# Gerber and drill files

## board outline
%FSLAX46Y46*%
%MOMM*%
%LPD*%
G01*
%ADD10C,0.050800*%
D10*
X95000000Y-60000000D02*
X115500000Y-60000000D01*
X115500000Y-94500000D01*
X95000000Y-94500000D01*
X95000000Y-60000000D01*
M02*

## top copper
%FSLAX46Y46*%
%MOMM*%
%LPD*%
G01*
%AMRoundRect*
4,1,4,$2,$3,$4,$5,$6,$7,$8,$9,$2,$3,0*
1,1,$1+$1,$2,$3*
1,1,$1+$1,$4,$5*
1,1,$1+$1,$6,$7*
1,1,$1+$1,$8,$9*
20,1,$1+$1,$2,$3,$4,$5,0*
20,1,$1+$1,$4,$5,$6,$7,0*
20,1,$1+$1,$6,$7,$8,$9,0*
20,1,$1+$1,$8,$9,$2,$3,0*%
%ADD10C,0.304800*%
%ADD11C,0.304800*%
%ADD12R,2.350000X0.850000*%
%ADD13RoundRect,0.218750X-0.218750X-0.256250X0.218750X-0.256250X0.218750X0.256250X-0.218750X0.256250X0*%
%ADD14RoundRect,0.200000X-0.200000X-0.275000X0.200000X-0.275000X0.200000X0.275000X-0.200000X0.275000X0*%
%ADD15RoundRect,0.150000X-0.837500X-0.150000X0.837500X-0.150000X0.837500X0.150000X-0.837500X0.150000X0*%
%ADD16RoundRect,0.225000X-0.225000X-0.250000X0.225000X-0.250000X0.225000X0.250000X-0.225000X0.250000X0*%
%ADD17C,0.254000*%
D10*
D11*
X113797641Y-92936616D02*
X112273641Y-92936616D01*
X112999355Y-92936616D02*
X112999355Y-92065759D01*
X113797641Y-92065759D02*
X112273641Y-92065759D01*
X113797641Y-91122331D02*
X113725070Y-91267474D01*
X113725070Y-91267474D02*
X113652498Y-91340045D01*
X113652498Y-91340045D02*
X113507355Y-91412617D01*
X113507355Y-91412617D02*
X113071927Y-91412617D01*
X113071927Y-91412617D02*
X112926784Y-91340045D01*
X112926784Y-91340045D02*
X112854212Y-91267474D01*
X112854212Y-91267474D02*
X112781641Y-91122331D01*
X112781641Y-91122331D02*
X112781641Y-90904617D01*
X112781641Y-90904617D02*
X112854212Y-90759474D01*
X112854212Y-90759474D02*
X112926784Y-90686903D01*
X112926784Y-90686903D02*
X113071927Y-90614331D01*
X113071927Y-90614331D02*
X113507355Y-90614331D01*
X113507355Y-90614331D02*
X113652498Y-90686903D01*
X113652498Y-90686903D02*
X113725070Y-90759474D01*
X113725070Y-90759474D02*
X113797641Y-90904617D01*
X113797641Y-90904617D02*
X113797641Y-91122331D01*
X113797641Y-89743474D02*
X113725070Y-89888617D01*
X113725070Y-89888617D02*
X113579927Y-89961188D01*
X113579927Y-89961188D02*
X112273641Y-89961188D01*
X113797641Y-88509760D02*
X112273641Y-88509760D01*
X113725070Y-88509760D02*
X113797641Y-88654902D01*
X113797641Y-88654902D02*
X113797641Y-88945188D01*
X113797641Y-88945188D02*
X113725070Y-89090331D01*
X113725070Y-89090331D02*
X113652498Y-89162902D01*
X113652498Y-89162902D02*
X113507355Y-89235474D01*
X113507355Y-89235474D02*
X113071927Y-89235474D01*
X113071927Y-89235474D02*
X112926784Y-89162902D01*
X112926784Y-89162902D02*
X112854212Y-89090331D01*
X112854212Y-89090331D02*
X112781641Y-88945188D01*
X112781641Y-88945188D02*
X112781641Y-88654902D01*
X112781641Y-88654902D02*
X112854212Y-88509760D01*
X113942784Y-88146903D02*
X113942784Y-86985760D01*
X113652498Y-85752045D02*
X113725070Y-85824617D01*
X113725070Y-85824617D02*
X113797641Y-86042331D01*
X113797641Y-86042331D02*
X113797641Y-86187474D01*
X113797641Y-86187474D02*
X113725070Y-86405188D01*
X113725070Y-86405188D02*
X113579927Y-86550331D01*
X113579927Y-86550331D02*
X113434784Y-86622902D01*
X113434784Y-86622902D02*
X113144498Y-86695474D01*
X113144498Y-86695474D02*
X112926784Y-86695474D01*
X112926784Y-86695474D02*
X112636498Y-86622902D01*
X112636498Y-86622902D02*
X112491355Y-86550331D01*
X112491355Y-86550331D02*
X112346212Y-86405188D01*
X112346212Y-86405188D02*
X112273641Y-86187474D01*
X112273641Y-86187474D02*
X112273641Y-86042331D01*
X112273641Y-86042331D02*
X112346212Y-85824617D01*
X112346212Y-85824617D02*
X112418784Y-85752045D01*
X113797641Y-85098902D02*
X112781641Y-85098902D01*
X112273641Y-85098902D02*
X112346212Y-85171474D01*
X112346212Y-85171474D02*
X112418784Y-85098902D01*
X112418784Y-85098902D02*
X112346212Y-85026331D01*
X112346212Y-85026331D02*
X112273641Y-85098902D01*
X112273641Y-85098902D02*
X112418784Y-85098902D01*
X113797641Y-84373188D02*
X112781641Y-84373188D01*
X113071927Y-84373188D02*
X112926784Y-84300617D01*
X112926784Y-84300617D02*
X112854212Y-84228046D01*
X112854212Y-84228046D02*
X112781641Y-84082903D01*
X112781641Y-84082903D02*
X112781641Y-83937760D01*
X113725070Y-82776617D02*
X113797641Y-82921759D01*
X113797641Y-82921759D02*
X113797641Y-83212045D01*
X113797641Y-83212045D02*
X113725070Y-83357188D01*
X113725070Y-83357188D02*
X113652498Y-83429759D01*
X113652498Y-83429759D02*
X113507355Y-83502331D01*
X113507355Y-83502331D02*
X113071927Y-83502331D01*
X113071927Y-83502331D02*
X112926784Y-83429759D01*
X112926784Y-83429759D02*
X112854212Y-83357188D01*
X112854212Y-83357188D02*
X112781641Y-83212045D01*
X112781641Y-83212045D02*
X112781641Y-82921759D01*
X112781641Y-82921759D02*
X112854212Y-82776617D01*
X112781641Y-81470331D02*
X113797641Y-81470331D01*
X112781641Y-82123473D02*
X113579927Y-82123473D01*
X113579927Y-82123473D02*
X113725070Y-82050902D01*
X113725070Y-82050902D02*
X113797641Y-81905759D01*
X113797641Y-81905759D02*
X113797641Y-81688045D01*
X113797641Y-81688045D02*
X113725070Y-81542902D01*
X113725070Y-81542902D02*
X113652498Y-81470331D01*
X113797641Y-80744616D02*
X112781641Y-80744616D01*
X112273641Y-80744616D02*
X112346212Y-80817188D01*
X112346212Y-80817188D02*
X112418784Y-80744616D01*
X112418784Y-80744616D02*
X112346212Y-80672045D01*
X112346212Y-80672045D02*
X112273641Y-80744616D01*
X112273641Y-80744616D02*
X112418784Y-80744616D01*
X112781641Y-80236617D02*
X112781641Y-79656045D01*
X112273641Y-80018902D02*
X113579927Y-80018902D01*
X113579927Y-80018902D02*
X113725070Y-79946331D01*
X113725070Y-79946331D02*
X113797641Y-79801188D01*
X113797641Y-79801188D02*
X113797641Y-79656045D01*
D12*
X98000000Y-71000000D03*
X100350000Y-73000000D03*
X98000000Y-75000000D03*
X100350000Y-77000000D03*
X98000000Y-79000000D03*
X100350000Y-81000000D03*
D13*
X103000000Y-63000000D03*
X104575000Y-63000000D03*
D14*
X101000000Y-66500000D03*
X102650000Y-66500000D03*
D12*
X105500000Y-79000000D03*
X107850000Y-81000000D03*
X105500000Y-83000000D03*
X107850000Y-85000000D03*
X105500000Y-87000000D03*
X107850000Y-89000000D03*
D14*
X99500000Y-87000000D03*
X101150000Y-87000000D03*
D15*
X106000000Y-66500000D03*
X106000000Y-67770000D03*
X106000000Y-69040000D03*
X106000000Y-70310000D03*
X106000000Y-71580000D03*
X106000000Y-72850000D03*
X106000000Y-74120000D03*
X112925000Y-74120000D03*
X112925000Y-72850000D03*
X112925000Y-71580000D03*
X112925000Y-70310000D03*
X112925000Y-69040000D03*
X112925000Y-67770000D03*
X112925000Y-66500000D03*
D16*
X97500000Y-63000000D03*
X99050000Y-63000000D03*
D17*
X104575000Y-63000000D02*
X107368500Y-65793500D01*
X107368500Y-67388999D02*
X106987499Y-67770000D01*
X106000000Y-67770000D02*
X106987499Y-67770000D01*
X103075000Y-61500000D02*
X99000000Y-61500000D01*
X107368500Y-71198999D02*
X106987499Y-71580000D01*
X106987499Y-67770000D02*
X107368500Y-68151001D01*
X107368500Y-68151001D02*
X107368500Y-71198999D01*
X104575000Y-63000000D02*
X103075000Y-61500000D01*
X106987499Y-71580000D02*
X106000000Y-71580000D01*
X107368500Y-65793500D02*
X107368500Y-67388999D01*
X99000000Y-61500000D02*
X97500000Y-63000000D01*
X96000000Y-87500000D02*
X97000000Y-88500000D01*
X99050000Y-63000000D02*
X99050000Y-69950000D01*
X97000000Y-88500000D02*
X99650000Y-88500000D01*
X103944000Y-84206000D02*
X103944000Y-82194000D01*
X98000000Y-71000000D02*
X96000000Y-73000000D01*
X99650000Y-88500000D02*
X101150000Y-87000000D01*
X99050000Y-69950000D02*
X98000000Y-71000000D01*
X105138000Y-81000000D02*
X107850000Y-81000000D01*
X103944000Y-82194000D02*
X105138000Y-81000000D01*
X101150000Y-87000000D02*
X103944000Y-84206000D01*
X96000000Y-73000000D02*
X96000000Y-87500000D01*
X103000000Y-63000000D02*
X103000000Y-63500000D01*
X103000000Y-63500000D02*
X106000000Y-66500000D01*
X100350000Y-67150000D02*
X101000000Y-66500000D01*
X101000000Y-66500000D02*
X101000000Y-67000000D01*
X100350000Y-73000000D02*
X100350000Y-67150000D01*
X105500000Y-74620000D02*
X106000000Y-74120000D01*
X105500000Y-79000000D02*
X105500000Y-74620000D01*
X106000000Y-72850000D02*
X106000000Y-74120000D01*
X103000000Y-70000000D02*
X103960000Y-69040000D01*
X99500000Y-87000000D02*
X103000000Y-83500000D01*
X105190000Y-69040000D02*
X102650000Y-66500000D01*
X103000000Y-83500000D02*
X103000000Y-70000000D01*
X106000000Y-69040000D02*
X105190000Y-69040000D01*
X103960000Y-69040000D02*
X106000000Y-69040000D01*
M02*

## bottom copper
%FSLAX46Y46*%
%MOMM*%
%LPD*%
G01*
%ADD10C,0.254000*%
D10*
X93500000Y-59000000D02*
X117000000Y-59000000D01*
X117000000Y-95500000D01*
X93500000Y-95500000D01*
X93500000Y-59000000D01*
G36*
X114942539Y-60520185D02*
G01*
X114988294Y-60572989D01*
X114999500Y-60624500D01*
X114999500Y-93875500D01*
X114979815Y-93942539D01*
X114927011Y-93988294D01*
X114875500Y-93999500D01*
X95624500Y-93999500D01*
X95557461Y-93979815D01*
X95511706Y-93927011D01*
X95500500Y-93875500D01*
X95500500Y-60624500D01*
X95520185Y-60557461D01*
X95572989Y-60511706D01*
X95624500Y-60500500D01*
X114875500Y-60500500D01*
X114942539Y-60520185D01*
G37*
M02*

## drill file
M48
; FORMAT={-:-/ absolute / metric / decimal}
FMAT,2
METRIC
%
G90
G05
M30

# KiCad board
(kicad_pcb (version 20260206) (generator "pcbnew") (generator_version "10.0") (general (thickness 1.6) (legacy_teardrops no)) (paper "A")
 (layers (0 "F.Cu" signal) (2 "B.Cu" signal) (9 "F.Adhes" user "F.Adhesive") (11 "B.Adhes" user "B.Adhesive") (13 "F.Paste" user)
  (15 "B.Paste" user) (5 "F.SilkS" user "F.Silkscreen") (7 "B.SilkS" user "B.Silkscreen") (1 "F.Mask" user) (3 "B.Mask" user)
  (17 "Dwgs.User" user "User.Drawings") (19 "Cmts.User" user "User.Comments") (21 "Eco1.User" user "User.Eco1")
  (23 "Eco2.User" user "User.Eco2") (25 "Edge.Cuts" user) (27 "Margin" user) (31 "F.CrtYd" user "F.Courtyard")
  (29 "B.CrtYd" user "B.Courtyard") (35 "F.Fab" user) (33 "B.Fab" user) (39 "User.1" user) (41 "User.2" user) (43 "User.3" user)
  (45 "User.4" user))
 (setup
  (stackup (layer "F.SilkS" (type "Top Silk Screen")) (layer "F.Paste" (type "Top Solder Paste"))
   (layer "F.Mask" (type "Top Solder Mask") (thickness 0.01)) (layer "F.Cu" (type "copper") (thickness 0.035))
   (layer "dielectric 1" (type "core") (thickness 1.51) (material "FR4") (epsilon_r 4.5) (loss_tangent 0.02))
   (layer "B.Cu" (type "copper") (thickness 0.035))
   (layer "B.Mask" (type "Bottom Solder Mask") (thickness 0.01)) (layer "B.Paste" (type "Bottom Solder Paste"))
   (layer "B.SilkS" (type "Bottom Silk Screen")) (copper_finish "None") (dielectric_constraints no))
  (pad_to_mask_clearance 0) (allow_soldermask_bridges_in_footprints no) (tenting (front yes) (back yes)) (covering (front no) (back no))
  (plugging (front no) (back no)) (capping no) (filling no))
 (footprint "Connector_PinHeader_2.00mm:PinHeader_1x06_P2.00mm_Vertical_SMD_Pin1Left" (layer "F.Cu") (at 99.175 76)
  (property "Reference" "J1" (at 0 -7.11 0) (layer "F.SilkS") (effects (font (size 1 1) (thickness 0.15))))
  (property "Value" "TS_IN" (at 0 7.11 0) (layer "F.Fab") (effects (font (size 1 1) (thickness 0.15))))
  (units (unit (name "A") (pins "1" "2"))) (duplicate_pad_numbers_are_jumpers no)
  (pad "1" smd rect (at -1.175 -5) (size 2.35 0.85) (layers "F.Cu" "F.Mask" "F.Paste") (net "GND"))
  (pad "2" smd rect (at 1.175 -3) (size 2.35 0.85) (layers "F.Cu" "F.Mask" "F.Paste") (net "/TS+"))
  (pad "3" smd rect (at -1.175 -1) (size 2.35 0.85) (layers "F.Cu" "F.Mask" "F.Paste"))
  (pad "4" smd rect (at 1.175 1) (size 2.35 0.85) (layers "F.Cu" "F.Mask" "F.Paste"))
  (pad "5" smd rect (at -1.175 3) (size 2.35 0.85) (layers "F.Cu" "F.Mask" "F.Paste"))
  (pad "6" smd rect (at 1.175 5) (size 2.35 0.85) (layers "F.Cu" "F.Mask" "F.Paste")))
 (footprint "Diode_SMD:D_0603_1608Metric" (layer "F.Cu") (at 103.7875 63)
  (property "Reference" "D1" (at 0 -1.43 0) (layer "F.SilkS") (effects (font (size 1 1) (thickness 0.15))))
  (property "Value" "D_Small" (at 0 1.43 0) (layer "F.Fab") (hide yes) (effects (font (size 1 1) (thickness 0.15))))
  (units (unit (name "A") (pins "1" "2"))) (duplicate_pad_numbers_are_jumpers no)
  (pad "1" smd roundrect (at -0.7875 0) (size 0.875 0.95) (layers "F.Cu" "F.Mask" "F.Paste") (roundrect_rratio 0.25) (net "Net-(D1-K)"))
  (pad "2" smd roundrect (at 0.7875 0) (size 0.875 0.95) (layers "F.Cu" "F.Mask" "F.Paste") (roundrect_rratio 0.25) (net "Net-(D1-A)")))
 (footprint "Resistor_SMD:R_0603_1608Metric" (layer "F.Cu") (at 101.825 66.5)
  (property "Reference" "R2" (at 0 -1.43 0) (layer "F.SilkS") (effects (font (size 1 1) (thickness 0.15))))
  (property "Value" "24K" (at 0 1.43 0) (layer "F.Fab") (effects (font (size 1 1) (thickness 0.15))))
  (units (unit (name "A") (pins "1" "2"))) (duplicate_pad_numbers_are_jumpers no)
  (pad "1" smd roundrect (at -0.825 0) (size 0.8 0.95) (layers "F.Cu" "F.Mask" "F.Paste") (roundrect_rratio 0.25) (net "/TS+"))
  (pad "2" smd roundrect (at 0.825 0) (size 0.8 0.95) (layers "F.Cu" "F.Mask" "F.Paste") (roundrect_rratio 0.25) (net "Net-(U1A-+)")))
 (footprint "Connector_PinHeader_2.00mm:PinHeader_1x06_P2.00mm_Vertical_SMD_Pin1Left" (layer "F.Cu") (at 106.675 84)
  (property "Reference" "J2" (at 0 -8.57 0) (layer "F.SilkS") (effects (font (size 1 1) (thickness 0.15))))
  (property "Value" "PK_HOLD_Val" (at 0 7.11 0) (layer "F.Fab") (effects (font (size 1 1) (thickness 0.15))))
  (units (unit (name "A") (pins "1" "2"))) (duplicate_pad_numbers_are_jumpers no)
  (pad "1" smd rect (at -1.175 -5) (size 2.35 0.85) (layers "F.Cu" "F.Mask" "F.Paste") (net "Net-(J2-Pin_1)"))
  (pad "2" smd rect (at 1.175 -3) (size 2.35 0.85) (layers "F.Cu" "F.Mask" "F.Paste") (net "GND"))
  (pad "3" smd rect (at -1.175 -1) (size 2.35 0.85) (layers "F.Cu" "F.Mask" "F.Paste"))
  (pad "4" smd rect (at 1.175 1) (size 2.35 0.85) (layers "F.Cu" "F.Mask" "F.Paste"))
  (pad "5" smd rect (at -1.175 3) (size 2.35 0.85) (layers "F.Cu" "F.Mask" "F.Paste"))
  (pad "6" smd rect (at 1.175 5) (size 2.35 0.85) (layers "F.Cu" "F.Mask" "F.Paste")))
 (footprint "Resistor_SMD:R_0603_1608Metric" (layer "F.Cu") (at 100.325 87)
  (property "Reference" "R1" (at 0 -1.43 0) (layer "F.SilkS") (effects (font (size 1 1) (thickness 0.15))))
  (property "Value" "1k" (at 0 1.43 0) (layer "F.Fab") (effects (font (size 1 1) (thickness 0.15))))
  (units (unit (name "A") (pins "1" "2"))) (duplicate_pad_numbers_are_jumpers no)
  (pad "1" smd roundrect (at -0.825 0) (size 0.8 0.95) (layers "F.Cu" "F.Mask" "F.Paste") (roundrect_rratio 0.25) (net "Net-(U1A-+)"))
  (pad "2" smd roundrect (at 0.825 0) (size 0.8 0.95) (layers "F.Cu" "F.Mask" "F.Paste") (roundrect_rratio 0.25) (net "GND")))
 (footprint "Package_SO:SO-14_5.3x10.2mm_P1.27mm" (layer "F.Cu") (at 109.4625 70.31)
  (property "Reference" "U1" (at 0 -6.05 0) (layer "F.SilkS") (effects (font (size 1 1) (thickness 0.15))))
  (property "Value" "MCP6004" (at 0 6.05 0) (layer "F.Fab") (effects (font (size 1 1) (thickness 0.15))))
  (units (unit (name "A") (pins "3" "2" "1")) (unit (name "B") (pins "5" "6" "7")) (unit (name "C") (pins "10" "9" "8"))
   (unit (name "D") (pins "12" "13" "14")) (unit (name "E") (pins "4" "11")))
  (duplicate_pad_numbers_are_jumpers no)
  (pad "1" smd roundrect (at -3.4625 -3.81) (size 1.975 0.6) (layers "F.Cu" "F.Mask" "F.Paste") (roundrect_rratio 0.25) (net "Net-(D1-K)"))
  (pad "2" smd roundrect (at -3.4625 -2.54) (size 1.975 0.6) (layers "F.Cu" "F.Mask" "F.Paste") (roundrect_rratio 0.25) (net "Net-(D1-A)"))
  (pad "3" smd roundrect (at -3.4625 -1.27) (size 1.975 0.6) (layers "F.Cu" "F.Mask" "F.Paste") (roundrect_rratio 0.25) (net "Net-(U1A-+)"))
  (pad "4" smd roundrect (at -3.4625 0) (size 1.975 0.6) (layers "F.Cu" "F.Mask" "F.Paste") (roundrect_rratio 0.25)
   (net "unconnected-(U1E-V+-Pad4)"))
  (pad "5" smd roundrect (at -3.4625 1.27) (size 1.975 0.6) (layers "F.Cu" "F.Mask" "F.Paste") (roundrect_rratio 0.25) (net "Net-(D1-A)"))
  (pad "6" smd roundrect (at -3.4625 2.54) (size 1.975 0.6) (layers "F.Cu" "F.Mask" "F.Paste") (roundrect_rratio 0.25)
   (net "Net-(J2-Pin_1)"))
  (pad "7" smd roundrect (at -3.4625 3.81) (size 1.975 0.6) (layers "F.Cu" "F.Mask" "F.Paste") (roundrect_rratio 0.25)
   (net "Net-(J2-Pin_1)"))
  (pad "8" smd roundrect (at 3.4625 3.81) (size 1.975 0.6) (layers "F.Cu" "F.Mask" "F.Paste") (roundrect_rratio 0.25)
   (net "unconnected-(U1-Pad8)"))
  (pad "9" smd roundrect (at 3.4625 2.54) (size 1.975 0.6) (layers "F.Cu" "F.Mask" "F.Paste") (roundrect_rratio 0.25)
   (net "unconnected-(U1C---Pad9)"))
  (pad "10" smd roundrect (at 3.4625 1.27) (size 1.975 0.6) (layers "F.Cu" "F.Mask" "F.Paste") (roundrect_rratio 0.25)
   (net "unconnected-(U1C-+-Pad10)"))
  (pad "11" smd roundrect (at 3.4625 0) (size 1.975 0.6) (layers "F.Cu" "F.Mask" "F.Paste") (roundrect_rratio 0.25)
   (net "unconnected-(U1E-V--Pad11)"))
  (pad "12" smd roundrect (at 3.4625 -1.27) (size 1.975 0.6) (layers "F.Cu" "F.Mask" "F.Paste") (roundrect_rratio 0.25)
   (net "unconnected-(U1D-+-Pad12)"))
  (pad "13" smd roundrect (at 3.4625 -2.54) (size 1.975 0.6) (layers "F.Cu" "F.Mask" "F.Paste") (roundrect_rratio 0.25)
   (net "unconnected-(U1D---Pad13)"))
  (pad "14" smd roundrect (at 3.4625 -3.81) (size 1.975 0.6) (layers "F.Cu" "F.Mask" "F.Paste") (roundrect_rratio 0.25)
   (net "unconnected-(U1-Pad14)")))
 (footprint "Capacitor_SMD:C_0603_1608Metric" (layer "F.Cu") (at 98.275 63)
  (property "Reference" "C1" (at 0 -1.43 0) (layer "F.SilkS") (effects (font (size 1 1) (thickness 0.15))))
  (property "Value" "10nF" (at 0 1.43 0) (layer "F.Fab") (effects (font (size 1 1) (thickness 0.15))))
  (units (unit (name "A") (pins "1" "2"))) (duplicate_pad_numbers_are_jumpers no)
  (pad "1" smd roundrect (at -0.775 0) (size 0.9 0.95) (layers "F.Cu" "F.Mask" "F.Paste") (roundrect_rratio 0.25) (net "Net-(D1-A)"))
  (pad "2" smd roundrect (at 0.775 0) (size 0.9 0.95) (layers "F.Cu" "F.Mask" "F.Paste") (roundrect_rratio 0.25) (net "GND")))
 (gr_rect (start 93.5 59) (end 117 95.5) (stroke (width 0.254) (type default)) (fill no) (layer "B.Cu"))
 (gr_rect (start 95 60) (end 115.5 94.5) (stroke (width 0.0508) (type default)) (fill no) (layer "Edge.Cuts"))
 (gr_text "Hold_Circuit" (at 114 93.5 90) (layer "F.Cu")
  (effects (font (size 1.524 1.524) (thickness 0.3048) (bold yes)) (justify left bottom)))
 (segment (start 104.575 63) (end 107.3685 65.7935) (width 0.254) (layer "F.Cu") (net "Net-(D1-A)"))
 (segment (start 107.3685 67.388999) (end 106.987499 67.77) (width 0.254) (layer "F.Cu") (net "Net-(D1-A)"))
 (segment (start 106 67.77) (end 106.987499 67.77) (width 0.254) (layer "F.Cu") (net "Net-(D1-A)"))
 (segment (start 103.075 61.5) (end 99 61.5) (width 0.254) (layer "F.Cu") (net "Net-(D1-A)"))
 (segment (start 107.3685 71.198999) (end 106.987499 71.58) (width 0.254) (layer "F.Cu") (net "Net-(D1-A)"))
 (segment (start 106.987499 67.77) (end 107.3685 68.151001) (width 0.254) (layer "F.Cu") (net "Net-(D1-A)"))
 (segment (start 107.3685 68.151001) (end 107.3685 71.198999) (width 0.254) (layer "F.Cu") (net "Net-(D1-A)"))
 (segment (start 104.575 63) (end 103.075 61.5) (width 0.254) (layer "F.Cu") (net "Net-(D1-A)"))
 (segment (start 106.987499 71.58) (end 106 71.58) (width 0.254) (layer "F.Cu") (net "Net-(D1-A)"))
 (segment (start 107.3685 65.7935) (end 107.3685 67.388999) (width 0.254) (layer "F.Cu") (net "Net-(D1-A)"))
 (segment (start 99 61.5) (end 97.5 63) (width 0.254) (layer "F.Cu") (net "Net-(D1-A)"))
 (segment (start 96 87.5) (end 97 88.5) (width 0.254) (layer "F.Cu") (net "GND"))
 (segment (start 99.05 63) (end 99.05 69.95) (width 0.254) (layer "F.Cu") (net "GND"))
 (segment (start 97 88.5) (end 99.65 88.5) (width 0.254) (layer "F.Cu") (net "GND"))
 (segment (start 103.944 84.206) (end 103.944 82.194) (width 0.254) (layer "F.Cu") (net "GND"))
 (segment (start 98 71) (end 96 73) (width 0.254) (layer "F.Cu") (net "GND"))
 (segment (start 99.65 88.5) (end 101.15 87) (width 0.254) (layer "F.Cu") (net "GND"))
 (segment (start 99.05 69.95) (end 98 71) (width 0.254) (layer "F.Cu") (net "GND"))
 (segment (start 105.138 81) (end 107.85 81) (width 0.254) (layer "F.Cu") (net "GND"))
 (segment (start 103.944 82.194) (end 105.138 81) (width 0.254) (layer "F.Cu") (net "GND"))
 (segment (start 101.15 87) (end 103.944 84.206) (width 0.254) (layer "F.Cu") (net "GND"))
 (segment (start 96 73) (end 96 87.5) (width 0.254) (layer "F.Cu") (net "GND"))
 (segment (start 103 63) (end 103 63.5) (width 0.254) (layer "F.Cu") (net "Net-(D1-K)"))
 (segment (start 103 63.5) (end 106 66.5) (width 0.254) (layer "F.Cu") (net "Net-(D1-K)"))
 (segment (start 100.35 67.15) (end 101 66.5) (width 0.254) (layer "F.Cu") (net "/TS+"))
 (segment (start 101 66.5) (end 101 67) (width 0.254) (layer "F.Cu") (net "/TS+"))
 (segment (start 100.35 73) (end 100.35 67.15) (width 0.254) (layer "F.Cu") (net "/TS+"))
 (segment (start 105.5 74.62) (end 106 74.12) (width 0.254) (layer "F.Cu") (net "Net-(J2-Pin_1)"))
 (segment (start 105.5 79) (end 105.5 74.62) (width 0.254) (layer "F.Cu") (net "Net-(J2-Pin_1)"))
 (segment (start 106 72.85) (end 106 74.12) (width 0.254) (layer "F.Cu") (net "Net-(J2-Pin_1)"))
 (segment (start 103 70) (end 103.96 69.04) (width 0.254) (layer "F.Cu") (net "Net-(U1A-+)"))
 (segment (start 99.5 87) (end 103 83.5) (width 0.254) (layer "F.Cu") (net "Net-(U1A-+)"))
 (segment (start 105.19 69.04) (end 102.65 66.5) (width 0.254) (layer "F.Cu") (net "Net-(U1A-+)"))
 (segment (start 103 83.5) (end 103 70) (width 0.254) (layer "F.Cu") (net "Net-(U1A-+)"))
 (segment (start 106 69.04) (end 105.19 69.04) (width 0.254) (layer "F.Cu") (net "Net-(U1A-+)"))
 (segment (start 103.96 69.04) (end 106 69.04) (width 0.254) (layer "F.Cu") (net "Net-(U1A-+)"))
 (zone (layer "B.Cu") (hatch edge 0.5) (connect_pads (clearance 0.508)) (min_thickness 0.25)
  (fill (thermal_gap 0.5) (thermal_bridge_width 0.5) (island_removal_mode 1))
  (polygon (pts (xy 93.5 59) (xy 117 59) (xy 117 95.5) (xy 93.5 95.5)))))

